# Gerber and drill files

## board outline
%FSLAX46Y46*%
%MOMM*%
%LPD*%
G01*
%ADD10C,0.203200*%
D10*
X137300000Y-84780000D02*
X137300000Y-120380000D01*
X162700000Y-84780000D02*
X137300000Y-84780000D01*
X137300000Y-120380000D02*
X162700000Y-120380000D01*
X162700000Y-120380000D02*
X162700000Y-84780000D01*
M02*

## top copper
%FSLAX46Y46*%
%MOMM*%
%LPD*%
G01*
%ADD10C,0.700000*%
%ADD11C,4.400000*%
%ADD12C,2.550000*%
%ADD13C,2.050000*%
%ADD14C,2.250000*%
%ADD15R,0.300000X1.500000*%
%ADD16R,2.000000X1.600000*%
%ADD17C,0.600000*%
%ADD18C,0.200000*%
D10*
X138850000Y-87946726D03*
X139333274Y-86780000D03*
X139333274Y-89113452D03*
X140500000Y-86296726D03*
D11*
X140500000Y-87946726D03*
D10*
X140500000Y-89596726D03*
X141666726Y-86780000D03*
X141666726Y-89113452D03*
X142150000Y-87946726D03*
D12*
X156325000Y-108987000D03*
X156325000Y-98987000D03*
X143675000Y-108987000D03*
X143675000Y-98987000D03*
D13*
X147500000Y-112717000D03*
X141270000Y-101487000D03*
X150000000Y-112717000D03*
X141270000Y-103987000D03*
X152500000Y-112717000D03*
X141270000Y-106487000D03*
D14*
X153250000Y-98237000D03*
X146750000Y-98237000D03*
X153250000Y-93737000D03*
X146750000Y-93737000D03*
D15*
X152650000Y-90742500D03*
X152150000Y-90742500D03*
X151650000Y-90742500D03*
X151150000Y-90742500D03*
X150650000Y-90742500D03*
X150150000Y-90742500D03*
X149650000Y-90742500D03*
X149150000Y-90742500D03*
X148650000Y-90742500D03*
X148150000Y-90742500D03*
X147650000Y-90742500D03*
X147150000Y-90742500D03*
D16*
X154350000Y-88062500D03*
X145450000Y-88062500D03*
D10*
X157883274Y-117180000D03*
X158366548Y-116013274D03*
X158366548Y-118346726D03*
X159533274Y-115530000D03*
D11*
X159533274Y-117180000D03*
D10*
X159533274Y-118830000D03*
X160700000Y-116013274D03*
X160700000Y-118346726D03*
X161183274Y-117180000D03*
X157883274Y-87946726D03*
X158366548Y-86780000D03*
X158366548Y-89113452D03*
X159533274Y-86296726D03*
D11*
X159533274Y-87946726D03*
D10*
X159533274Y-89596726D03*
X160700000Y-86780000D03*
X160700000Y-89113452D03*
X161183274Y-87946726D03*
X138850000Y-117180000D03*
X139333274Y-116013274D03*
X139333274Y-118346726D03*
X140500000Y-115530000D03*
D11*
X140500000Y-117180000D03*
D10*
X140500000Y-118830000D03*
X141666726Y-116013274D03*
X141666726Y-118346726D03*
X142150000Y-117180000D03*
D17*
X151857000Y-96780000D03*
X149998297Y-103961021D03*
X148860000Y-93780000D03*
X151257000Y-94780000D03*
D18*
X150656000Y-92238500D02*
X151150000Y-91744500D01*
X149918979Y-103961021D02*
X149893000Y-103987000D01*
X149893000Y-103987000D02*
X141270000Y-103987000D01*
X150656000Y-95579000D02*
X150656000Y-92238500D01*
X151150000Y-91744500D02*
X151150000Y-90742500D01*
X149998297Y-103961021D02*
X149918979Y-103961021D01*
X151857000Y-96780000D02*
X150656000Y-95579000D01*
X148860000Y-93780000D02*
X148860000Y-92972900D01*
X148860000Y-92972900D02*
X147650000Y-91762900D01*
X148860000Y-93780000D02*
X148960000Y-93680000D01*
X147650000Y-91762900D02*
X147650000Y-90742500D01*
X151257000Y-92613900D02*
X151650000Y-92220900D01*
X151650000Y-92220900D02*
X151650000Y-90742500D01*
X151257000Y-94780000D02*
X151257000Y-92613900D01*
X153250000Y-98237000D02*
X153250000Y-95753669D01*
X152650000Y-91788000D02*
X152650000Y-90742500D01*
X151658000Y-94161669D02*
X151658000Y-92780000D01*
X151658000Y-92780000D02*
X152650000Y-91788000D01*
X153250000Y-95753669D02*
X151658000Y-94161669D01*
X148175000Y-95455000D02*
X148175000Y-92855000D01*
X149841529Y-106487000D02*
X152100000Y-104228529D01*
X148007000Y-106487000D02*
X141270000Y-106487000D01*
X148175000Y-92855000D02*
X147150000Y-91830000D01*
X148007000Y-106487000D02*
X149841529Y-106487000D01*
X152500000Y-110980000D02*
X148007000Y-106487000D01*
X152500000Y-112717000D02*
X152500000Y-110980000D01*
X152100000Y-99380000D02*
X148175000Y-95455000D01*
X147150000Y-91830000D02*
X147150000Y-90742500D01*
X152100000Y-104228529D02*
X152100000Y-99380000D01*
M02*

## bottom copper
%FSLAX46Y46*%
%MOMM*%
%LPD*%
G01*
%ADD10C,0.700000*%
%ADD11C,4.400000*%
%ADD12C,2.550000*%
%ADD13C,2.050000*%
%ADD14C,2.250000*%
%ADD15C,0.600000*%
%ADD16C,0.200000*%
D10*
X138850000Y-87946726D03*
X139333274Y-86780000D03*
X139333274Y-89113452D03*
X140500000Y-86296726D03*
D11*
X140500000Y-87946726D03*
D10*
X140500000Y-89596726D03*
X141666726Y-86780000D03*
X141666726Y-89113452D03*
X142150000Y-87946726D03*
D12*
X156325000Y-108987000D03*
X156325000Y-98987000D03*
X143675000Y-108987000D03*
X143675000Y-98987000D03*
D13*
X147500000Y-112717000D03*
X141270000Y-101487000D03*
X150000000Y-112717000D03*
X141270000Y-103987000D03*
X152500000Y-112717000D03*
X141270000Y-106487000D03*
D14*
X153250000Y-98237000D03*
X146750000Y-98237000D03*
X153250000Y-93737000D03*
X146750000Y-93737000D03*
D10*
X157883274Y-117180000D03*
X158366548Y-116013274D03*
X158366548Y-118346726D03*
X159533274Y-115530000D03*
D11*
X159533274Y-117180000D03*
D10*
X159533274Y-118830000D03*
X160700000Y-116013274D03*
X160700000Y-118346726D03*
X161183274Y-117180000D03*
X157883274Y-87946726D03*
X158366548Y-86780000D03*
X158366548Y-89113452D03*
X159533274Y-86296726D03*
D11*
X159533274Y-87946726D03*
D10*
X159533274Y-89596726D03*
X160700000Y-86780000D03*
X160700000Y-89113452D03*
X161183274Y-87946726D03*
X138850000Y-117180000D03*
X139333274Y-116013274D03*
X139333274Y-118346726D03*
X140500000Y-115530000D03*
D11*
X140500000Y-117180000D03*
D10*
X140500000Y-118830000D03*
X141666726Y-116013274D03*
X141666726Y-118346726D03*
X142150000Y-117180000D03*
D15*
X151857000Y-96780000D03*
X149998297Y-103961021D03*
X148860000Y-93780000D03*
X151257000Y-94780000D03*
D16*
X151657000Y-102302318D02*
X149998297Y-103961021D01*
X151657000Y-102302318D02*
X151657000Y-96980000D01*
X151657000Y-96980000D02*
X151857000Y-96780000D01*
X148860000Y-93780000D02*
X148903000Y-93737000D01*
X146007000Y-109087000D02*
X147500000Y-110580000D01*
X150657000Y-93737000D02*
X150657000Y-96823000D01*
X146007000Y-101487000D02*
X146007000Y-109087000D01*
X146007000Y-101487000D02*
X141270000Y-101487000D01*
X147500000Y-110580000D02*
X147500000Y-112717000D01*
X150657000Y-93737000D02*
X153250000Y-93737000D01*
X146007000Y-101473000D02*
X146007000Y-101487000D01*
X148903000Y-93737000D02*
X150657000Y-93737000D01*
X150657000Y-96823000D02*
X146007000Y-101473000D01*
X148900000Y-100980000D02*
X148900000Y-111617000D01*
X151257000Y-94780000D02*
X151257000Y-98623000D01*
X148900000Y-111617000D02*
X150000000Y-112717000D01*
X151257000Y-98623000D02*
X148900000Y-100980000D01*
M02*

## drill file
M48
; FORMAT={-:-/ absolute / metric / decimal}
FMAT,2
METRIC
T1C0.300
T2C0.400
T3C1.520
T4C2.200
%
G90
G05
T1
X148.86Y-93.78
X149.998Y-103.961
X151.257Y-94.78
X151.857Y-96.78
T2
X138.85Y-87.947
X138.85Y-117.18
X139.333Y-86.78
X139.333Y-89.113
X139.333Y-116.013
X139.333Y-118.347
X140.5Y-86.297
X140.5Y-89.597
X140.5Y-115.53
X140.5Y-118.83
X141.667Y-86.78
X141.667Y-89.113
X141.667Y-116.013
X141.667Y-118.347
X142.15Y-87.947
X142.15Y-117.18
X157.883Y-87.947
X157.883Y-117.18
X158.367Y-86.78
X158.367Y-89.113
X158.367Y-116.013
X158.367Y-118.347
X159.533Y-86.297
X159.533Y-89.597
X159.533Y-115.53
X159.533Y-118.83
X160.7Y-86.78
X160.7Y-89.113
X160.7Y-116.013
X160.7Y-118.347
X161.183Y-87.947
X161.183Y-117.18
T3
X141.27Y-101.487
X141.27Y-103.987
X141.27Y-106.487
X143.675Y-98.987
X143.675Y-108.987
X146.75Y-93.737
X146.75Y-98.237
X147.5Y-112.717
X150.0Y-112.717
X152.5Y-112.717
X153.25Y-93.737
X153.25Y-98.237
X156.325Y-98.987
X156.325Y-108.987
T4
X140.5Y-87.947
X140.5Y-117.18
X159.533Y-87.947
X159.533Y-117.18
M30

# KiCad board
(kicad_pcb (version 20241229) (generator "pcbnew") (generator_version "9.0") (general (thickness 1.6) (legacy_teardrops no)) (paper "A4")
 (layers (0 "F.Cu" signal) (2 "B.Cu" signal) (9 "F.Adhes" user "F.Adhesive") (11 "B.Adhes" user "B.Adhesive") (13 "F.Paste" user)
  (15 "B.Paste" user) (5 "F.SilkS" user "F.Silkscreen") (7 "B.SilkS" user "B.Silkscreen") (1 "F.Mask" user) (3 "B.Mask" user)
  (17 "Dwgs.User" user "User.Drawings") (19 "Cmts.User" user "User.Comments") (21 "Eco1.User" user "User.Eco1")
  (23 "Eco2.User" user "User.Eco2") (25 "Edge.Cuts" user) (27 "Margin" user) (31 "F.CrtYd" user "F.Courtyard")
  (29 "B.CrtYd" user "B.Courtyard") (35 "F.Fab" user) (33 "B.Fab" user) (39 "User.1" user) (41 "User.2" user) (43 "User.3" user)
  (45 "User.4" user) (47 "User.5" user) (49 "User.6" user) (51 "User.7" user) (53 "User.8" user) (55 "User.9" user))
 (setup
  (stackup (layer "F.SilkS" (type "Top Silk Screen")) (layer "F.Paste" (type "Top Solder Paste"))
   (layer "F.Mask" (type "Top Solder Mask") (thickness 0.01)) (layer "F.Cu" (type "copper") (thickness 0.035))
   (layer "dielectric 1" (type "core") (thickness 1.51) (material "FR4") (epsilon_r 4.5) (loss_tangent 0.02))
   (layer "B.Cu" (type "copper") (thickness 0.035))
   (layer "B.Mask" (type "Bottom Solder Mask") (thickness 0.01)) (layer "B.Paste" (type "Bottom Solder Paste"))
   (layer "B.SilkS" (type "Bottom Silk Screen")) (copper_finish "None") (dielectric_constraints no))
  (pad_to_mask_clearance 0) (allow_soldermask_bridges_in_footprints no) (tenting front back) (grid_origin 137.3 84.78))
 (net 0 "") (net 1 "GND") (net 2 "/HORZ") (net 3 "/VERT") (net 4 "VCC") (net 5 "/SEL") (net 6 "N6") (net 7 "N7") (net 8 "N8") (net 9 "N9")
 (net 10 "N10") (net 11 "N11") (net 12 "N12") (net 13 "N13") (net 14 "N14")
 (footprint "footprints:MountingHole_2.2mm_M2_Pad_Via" (layer "F.Cu") (at 140.5 87.946726)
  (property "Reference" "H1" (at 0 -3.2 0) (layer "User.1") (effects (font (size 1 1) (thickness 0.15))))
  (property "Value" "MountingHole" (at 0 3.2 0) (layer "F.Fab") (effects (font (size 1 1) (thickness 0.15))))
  (pad "1" thru_hole circle (at -1.65 0) (size 0.7 0.7) (drill 0.4) (layers "*.Cu" "*.Mask") (remove_unused_layers no) (zone_connect 2))
  (pad "1" thru_hole circle (at -1.166726 -1.166726) (size 0.7 0.7) (drill 0.4) (layers "*.Cu" "*.Mask") (remove_unused_layers no)
   (zone_connect 2))
  (pad "1" thru_hole circle (at -1.166726 1.166726) (size 0.7 0.7) (drill 0.4) (layers "*.Cu" "*.Mask") (remove_unused_layers no)
   (zone_connect 2))
  (pad "1" thru_hole circle (at 0 -1.65) (size 0.7 0.7) (drill 0.4) (layers "*.Cu" "*.Mask") (remove_unused_layers no) (zone_connect 2))
  (pad "1" thru_hole circle (at 0 0) (size 4.4 4.4) (drill 2.2) (layers "*.Cu" "*.Mask") (remove_unused_layers no))
  (pad "1" thru_hole circle (at 0 1.65) (size 0.7 0.7) (drill 0.4) (layers "*.Cu" "*.Mask") (remove_unused_layers no) (zone_connect 2))
  (pad "1" thru_hole circle (at 1.166726 -1.166726) (size 0.7 0.7) (drill 0.4) (layers "*.Cu" "*.Mask") (remove_unused_layers no)
   (zone_connect 2))
  (pad "1" thru_hole circle (at 1.166726 1.166726) (size 0.7 0.7) (drill 0.4) (layers "*.Cu" "*.Mask") (remove_unused_layers no)
   (zone_connect 2))
  (pad "1" thru_hole circle (at 1.65 0) (size 0.7 0.7) (drill 0.4) (layers "*.Cu" "*.Mask") (remove_unused_layers no) (zone_connect 2)))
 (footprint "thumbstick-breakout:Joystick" (layer "F.Cu") (at 150 103.987 180)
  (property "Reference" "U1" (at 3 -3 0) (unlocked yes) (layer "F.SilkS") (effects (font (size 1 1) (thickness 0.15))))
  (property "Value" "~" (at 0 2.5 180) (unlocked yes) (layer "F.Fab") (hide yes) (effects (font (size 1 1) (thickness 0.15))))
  (pad "" thru_hole circle (at -6.325 -5 180) (size 2.55 2.55) (drill 1.52) (layers "*.Cu" "*.Mask") (remove_unused_layers no)
   (solder_mask_margin 0.1))
  (pad "" thru_hole circle (at -6.325 5 180) (size 2.55 2.55) (drill 1.52) (layers "*.Cu" "*.Mask") (remove_unused_layers no)
   (solder_mask_margin 0.1))
  (pad "" thru_hole circle (at 6.325 -5 180) (size 2.55 2.55) (drill 1.52) (layers "*.Cu" "*.Mask") (remove_unused_layers no)
   (solder_mask_margin 0.1))
  (pad "" thru_hole circle (at 6.325 5 180) (size 2.55 2.55) (drill 1.52) (layers "*.Cu" "*.Mask") (remove_unused_layers no)
   (solder_mask_margin 0.1))
  (pad "1" thru_hole circle (at 2.5 -8.73 180) (size 2.05 2.05) (drill 1.52) (layers "*.Cu" "*.Mask") (remove_unused_layers no)
   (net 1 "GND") (solder_mask_margin 0.1))
  (pad "1'" thru_hole circle (at 8.73 2.5 180) (size 2.05 2.05) (drill 1.52) (layers "*.Cu" "*.Mask") (remove_unused_layers no)
   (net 1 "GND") (solder_mask_margin 0.1))
  (pad "2" thru_hole circle (at 0 -8.73 180) (size 2.05 2.05) (drill 1.52) (layers "*.Cu" "*.Mask") (remove_unused_layers no)
   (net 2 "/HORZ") (solder_mask_margin 0.1))
  (pad "2'" thru_hole circle (at 8.73 0 180) (size 2.05 2.05) (drill 1.52) (layers "*.Cu" "*.Mask") (remove_unused_layers no)
   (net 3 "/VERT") (solder_mask_margin 0.1))
  (pad "3" thru_hole circle (at -2.5 -8.73 180) (size 2.05 2.05) (drill 1.52) (layers "*.Cu" "*.Mask") (remove_unused_layers no)
   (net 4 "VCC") (solder_mask_margin 0.1))
  (pad "3'" thru_hole circle (at 8.73 -2.5 180) (size 2.05 2.05) (drill 1.52) (layers "*.Cu" "*.Mask") (remove_unused_layers no)
   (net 4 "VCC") (solder_mask_margin 0.1))
  (pad "a" thru_hole circle (at -3.25 5.75 180) (size 2.25 2.25) (drill 1.52) (layers "*.Cu" "*.Mask") (remove_unused_layers no)
   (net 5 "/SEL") (solder_mask_margin 0.1))
  (pad "b" thru_hole circle (at 3.25 5.75 180) (size 2.25 2.25) (drill 1.52) (layers "*.Cu" "*.Mask") (remove_unused_layers no)
   (solder_mask_margin 0.1))
  (pad "c" thru_hole circle (at -3.25 10.25 180) (size 2.25 2.25) (drill 1.52) (layers "*.Cu" "*.Mask") (remove_unused_layers no)
   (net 1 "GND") (solder_mask_margin 0.1))
  (pad "d" thru_hole circle (at 3.25 10.25 180) (size 2.25 2.25) (drill 1.52) (layers "*.Cu" "*.Mask") (remove_unused_layers no)
   (solder_mask_margin 0.1)))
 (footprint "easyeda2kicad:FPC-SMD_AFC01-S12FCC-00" (layer "F.Cu") (at 149.9 89.4025 180)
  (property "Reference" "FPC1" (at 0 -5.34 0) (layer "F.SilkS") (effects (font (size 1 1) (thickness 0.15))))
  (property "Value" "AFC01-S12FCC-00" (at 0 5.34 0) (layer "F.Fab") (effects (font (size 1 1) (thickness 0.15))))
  (pad "1" smd rect (at -2.75 -1.34 180) (size 0.3 1.5) (layers "F.Cu" "F.Mask" "F.Paste") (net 5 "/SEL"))
  (pad "2" smd rect (at -2.25 -1.34 180) (size 0.3 1.5) (layers "F.Cu" "F.Mask" "F.Paste") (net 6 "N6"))
  (pad "3" smd rect (at -1.75 -1.34 180) (size 0.3 1.5) (layers "F.Cu" "F.Mask" "F.Paste") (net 2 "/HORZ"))
  (pad "4" smd rect (at -1.25 -1.34 180) (size 0.3 1.5) (layers "F.Cu" "F.Mask" "F.Paste") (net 3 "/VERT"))
  (pad "5" smd rect (at -0.75 -1.34 180) (size 0.3 1.5) (layers "F.Cu" "F.Mask" "F.Paste") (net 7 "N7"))
  (pad "6" smd rect (at -0.25 -1.34 180) (size 0.3 1.5) (layers "F.Cu" "F.Mask" "F.Paste") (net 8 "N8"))
  (pad "7" smd rect (at 0.25 -1.34 180) (size 0.3 1.5) (layers "F.Cu" "F.Mask" "F.Paste") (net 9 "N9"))
  (pad "8" smd rect (at 0.75 -1.34 180) (size 0.3 1.5) (layers "F.Cu" "F.Mask" "F.Paste") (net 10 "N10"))
  (pad "9" smd rect (at 1.25 -1.34 180) (size 0.3 1.5) (layers "F.Cu" "F.Mask" "F.Paste") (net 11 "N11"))
  (pad "10" smd rect (at 1.75 -1.34 180) (size 0.3 1.5) (layers "F.Cu" "F.Mask" "F.Paste") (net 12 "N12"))
  (pad "11" smd rect (at 2.25 -1.34 180) (size 0.3 1.5) (layers "F.Cu" "F.Mask" "F.Paste") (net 1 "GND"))
  (pad "12" smd rect (at 2.75 -1.34 180) (size 0.3 1.5) (layers "F.Cu" "F.Mask" "F.Paste") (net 4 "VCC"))
  (pad "13" smd rect (at -4.45 1.34 180) (size 2 1.6) (layers "F.Cu" "F.Mask" "F.Paste") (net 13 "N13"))
  (pad "14" smd rect (at 4.45 1.34) (size 2 1.6) (layers "F.Cu" "F.Mask" "F.Paste") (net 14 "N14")))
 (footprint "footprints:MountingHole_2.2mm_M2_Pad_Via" (layer "F.Cu") (at 159.533274 117.18)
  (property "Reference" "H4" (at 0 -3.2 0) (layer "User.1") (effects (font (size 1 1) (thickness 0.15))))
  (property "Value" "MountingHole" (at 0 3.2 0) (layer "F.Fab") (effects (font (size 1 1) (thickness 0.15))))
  (pad "1" thru_hole circle (at -1.65 0) (size 0.7 0.7) (drill 0.4) (layers "*.Cu" "*.Mask") (remove_unused_layers no) (zone_connect 2))
  (pad "1" thru_hole circle (at -1.166726 -1.166726) (size 0.7 0.7) (drill 0.4) (layers "*.Cu" "*.Mask") (remove_unused_layers no)
   (zone_connect 2))
  (pad "1" thru_hole circle (at -1.166726 1.166726) (size 0.7 0.7) (drill 0.4) (layers "*.Cu" "*.Mask") (remove_unused_layers no)
   (zone_connect 2))
  (pad "1" thru_hole circle (at 0 -1.65) (size 0.7 0.7) (drill 0.4) (layers "*.Cu" "*.Mask") (remove_unused_layers no) (zone_connect 2))
  (pad "1" thru_hole circle (at 0 0) (size 4.4 4.4) (drill 2.2) (layers "*.Cu" "*.Mask") (remove_unused_layers no))
  (pad "1" thru_hole circle (at 0 1.65) (size 0.7 0.7) (drill 0.4) (layers "*.Cu" "*.Mask") (remove_unused_layers no) (zone_connect 2))
  (pad "1" thru_hole circle (at 1.166726 -1.166726) (size 0.7 0.7) (drill 0.4) (layers "*.Cu" "*.Mask") (remove_unused_layers no)
   (zone_connect 2))
  (pad "1" thru_hole circle (at 1.166726 1.166726) (size 0.7 0.7) (drill 0.4) (layers "*.Cu" "*.Mask") (remove_unused_layers no)
   (zone_connect 2))
  (pad "1" thru_hole circle (at 1.65 0) (size 0.7 0.7) (drill 0.4) (layers "*.Cu" "*.Mask") (remove_unused_layers no) (zone_connect 2)))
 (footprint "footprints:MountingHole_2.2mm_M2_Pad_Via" (layer "F.Cu") (at 159.533274 87.946726)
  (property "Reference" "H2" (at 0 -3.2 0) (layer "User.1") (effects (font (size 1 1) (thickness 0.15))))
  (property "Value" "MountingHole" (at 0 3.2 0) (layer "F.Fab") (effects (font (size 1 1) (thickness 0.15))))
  (pad "1" thru_hole circle (at -1.65 0) (size 0.7 0.7) (drill 0.4) (layers "*.Cu" "*.Mask") (remove_unused_layers no) (zone_connect 2))
  (pad "1" thru_hole circle (at -1.166726 -1.166726) (size 0.7 0.7) (drill 0.4) (layers "*.Cu" "*.Mask") (remove_unused_layers no)
   (zone_connect 2))
  (pad "1" thru_hole circle (at -1.166726 1.166726) (size 0.7 0.7) (drill 0.4) (layers "*.Cu" "*.Mask") (remove_unused_layers no)
   (zone_connect 2))
  (pad "1" thru_hole circle (at 0 -1.65) (size 0.7 0.7) (drill 0.4) (layers "*.Cu" "*.Mask") (remove_unused_layers no) (zone_connect 2))
  (pad "1" thru_hole circle (at 0 0) (size 4.4 4.4) (drill 2.2) (layers "*.Cu" "*.Mask") (remove_unused_layers no))
  (pad "1" thru_hole circle (at 0 1.65) (size 0.7 0.7) (drill 0.4) (layers "*.Cu" "*.Mask") (remove_unused_layers no) (zone_connect 2))
  (pad "1" thru_hole circle (at 1.166726 -1.166726) (size 0.7 0.7) (drill 0.4) (layers "*.Cu" "*.Mask") (remove_unused_layers no)
   (zone_connect 2))
  (pad "1" thru_hole circle (at 1.166726 1.166726) (size 0.7 0.7) (drill 0.4) (layers "*.Cu" "*.Mask") (remove_unused_layers no)
   (zone_connect 2))
  (pad "1" thru_hole circle (at 1.65 0) (size 0.7 0.7) (drill 0.4) (layers "*.Cu" "*.Mask") (remove_unused_layers no) (zone_connect 2)))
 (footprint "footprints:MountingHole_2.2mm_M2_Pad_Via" (layer "F.Cu") (at 140.5 117.18)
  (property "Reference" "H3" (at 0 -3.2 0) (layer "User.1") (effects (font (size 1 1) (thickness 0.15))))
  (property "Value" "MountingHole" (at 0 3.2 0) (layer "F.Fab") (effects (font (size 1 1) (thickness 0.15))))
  (pad "1" thru_hole circle (at -1.65 0) (size 0.7 0.7) (drill 0.4) (layers "*.Cu" "*.Mask") (remove_unused_layers no) (zone_connect 2))
  (pad "1" thru_hole circle (at -1.166726 -1.166726) (size 0.7 0.7) (drill 0.4) (layers "*.Cu" "*.Mask") (remove_unused_layers no)
   (zone_connect 2))
  (pad "1" thru_hole circle (at -1.166726 1.166726) (size 0.7 0.7) (drill 0.4) (layers "*.Cu" "*.Mask") (remove_unused_layers no)
   (zone_connect 2))
  (pad "1" thru_hole circle (at 0 -1.65) (size 0.7 0.7) (drill 0.4) (layers "*.Cu" "*.Mask") (remove_unused_layers no) (zone_connect 2))
  (pad "1" thru_hole circle (at 0 0) (size 4.4 4.4) (drill 2.2) (layers "*.Cu" "*.Mask") (remove_unused_layers no))
  (pad "1" thru_hole circle (at 0 1.65) (size 0.7 0.7) (drill 0.4) (layers "*.Cu" "*.Mask") (remove_unused_layers no) (zone_connect 2))
  (pad "1" thru_hole circle (at 1.166726 -1.166726) (size 0.7 0.7) (drill 0.4) (layers "*.Cu" "*.Mask") (remove_unused_layers no)
   (zone_connect 2))
  (pad "1" thru_hole circle (at 1.166726 1.166726) (size 0.7 0.7) (drill 0.4) (layers "*.Cu" "*.Mask") (remove_unused_layers no)
   (zone_connect 2))
  (pad "1" thru_hole circle (at 1.65 0) (size 0.7 0.7) (drill 0.4) (layers "*.Cu" "*.Mask") (remove_unused_layers no) (zone_connect 2)))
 (gr_line (start 137.3 84.78) (end 137.3 120.38) (stroke (width 0.2032) (type solid)) (layer "Edge.Cuts"))
 (gr_line (start 162.7 84.78) (end 137.3 84.78) (stroke (width 0.2032) (type solid)) (layer "Edge.Cuts"))
 (gr_line (start 137.3 120.38) (end 162.7 120.38) (stroke (width 0.2032) (type solid)) (layer "Edge.Cuts"))
 (gr_line (start 162.7 120.38) (end 162.7 84.78) (stroke (width 0.2032) (type solid)) (layer "Edge.Cuts"))
 (segment (start 150.656 92.2385) (end 151.15 91.7445) (width 0.2) (layer "F.Cu") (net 3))
 (segment (start 149.918979 103.961021) (end 149.893 103.987) (width 0.2) (layer "F.Cu") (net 3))
 (segment (start 149.893 103.987) (end 141.27 103.987) (width 0.2) (layer "F.Cu") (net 3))
 (segment (start 150.656 95.579) (end 150.656 92.2385) (width 0.2) (layer "F.Cu") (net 3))
 (segment (start 151.15 91.7445) (end 151.15 90.7425) (width 0.2) (layer "F.Cu") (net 3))
 (segment (start 149.998297 103.961021) (end 149.918979 103.961021) (width 0.2) (layer "F.Cu") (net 3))
 (segment (start 151.857 96.78) (end 150.656 95.579) (width 0.2) (layer "F.Cu") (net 3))
 (via (at 151.857 96.78) (size 0.6) (drill 0.3) (layers "F.Cu" "B.Cu") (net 3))
 (via (at 149.998297 103.961021) (size 0.6) (drill 0.3) (layers "F.Cu" "B.Cu") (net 3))
 (segment (start 151.657 102.302318) (end 149.998297 103.961021) (width 0.2) (layer "B.Cu") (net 3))
 (segment (start 151.657 102.302318) (end 151.657 96.98) (width 0.2) (layer "B.Cu") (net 3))
 (segment (start 151.657 96.98) (end 151.857 96.78) (width 0.2) (layer "B.Cu") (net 3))
 (segment (start 148.86 93.78) (end 148.86 92.9729) (width 0.2) (layer "F.Cu") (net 1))
 (segment (start 148.86 92.9729) (end 147.65 91.7629) (width 0.2) (layer "F.Cu") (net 1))
 (segment (start 148.86 93.78) (end 148.96 93.68) (width 0.2) (layer "F.Cu") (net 1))
 (segment (start 147.65 91.7629) (end 147.65 90.7425) (width 0.2) (layer "F.Cu") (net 1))
 (via (at 148.86 93.78) (size 0.6) (drill 0.3) (layers "F.Cu" "B.Cu") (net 1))
 (segment (start 148.86 93.78) (end 148.903 93.737) (width 0.2) (layer "B.Cu") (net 1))
 (segment (start 146.007 109.087) (end 147.5 110.58) (width 0.2) (layer "B.Cu") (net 1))
 (segment (start 150.657 93.737) (end 150.657 96.823) (width 0.2) (layer "B.Cu") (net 1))
 (segment (start 146.007 101.487) (end 146.007 109.087) (width 0.2) (layer "B.Cu") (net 1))
 (segment (start 146.007 101.487) (end 141.27 101.487) (width 0.2) (layer "B.Cu") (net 1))
 (segment (start 147.5 110.58) (end 147.5 112.717) (width 0.2) (layer "B.Cu") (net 1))
 (segment (start 150.657 93.737) (end 153.25 93.737) (width 0.2) (layer "B.Cu") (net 1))
 (segment (start 146.007 101.473) (end 146.007 101.487) (width 0.2) (layer "B.Cu") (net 1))
 (segment (start 148.903 93.737) (end 150.657 93.737) (width 0.2) (layer "B.Cu") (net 1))
 (segment (start 150.657 96.823) (end 146.007 101.473) (width 0.2) (layer "B.Cu") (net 1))
 (segment (start 151.257 92.6139) (end 151.65 92.2209) (width 0.2) (layer "F.Cu") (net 2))
 (segment (start 151.65 92.2209) (end 151.65 90.7425) (width 0.2) (layer "F.Cu") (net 2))
 (segment (start 151.257 94.78) (end 151.257 92.6139) (width 0.2) (layer "F.Cu") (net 2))
 (via (at 151.257 94.78) (size 0.6) (drill 0.3) (layers "F.Cu" "B.Cu") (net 2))
 (segment (start 148.9 100.98) (end 148.9 111.617) (width 0.2) (layer "B.Cu") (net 2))
 (segment (start 151.257 94.78) (end 151.257 98.623) (width 0.2) (layer "B.Cu") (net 2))
 (segment (start 148.9 111.617) (end 150 112.717) (width 0.2) (layer "B.Cu") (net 2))
 (segment (start 151.257 98.623) (end 148.9 100.98) (width 0.2) (layer "B.Cu") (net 2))
 (segment (start 153.25 98.237) (end 153.25 95.753669) (width 0.2) (layer "F.Cu") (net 5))
 (segment (start 152.65 91.788) (end 152.65 90.7425) (width 0.2) (layer "F.Cu") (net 5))
 (segment (start 151.658 94.161669) (end 151.658 92.78) (width 0.2) (layer "F.Cu") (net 5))
 (segment (start 151.658 92.78) (end 152.65 91.788) (width 0.2) (layer "F.Cu") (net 5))
 (segment (start 153.25 95.753669) (end 151.658 94.161669) (width 0.2) (layer "F.Cu") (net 5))
 (segment (start 148.175 95.455) (end 148.175 92.855) (width 0.2) (layer "F.Cu") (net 4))
 (segment (start 149.841529 106.487) (end 152.1 104.228529) (width 0.2) (layer "F.Cu") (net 4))
 (segment (start 148.007 106.487) (end 141.27 106.487) (width 0.2) (layer "F.Cu") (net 4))
 (segment (start 148.175 92.855) (end 147.15 91.83) (width 0.2) (layer "F.Cu") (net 4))
 (segment (start 148.007 106.487) (end 149.841529 106.487) (width 0.2) (layer "F.Cu") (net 4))
 (segment (start 152.5 110.98) (end 148.007 106.487) (width 0.2) (layer "F.Cu") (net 4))
 (segment (start 152.5 112.717) (end 152.5 110.98) (width 0.2) (layer "F.Cu") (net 4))
 (segment (start 152.1 99.38) (end 148.175 95.455) (width 0.2) (layer "F.Cu") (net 4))
 (segment (start 147.15 91.83) (end 147.15 90.7425) (width 0.2) (layer "F.Cu") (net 4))
 (segment (start 152.1 104.228529) (end 152.1 99.38) (width 0.2) (layer "F.Cu") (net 4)))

